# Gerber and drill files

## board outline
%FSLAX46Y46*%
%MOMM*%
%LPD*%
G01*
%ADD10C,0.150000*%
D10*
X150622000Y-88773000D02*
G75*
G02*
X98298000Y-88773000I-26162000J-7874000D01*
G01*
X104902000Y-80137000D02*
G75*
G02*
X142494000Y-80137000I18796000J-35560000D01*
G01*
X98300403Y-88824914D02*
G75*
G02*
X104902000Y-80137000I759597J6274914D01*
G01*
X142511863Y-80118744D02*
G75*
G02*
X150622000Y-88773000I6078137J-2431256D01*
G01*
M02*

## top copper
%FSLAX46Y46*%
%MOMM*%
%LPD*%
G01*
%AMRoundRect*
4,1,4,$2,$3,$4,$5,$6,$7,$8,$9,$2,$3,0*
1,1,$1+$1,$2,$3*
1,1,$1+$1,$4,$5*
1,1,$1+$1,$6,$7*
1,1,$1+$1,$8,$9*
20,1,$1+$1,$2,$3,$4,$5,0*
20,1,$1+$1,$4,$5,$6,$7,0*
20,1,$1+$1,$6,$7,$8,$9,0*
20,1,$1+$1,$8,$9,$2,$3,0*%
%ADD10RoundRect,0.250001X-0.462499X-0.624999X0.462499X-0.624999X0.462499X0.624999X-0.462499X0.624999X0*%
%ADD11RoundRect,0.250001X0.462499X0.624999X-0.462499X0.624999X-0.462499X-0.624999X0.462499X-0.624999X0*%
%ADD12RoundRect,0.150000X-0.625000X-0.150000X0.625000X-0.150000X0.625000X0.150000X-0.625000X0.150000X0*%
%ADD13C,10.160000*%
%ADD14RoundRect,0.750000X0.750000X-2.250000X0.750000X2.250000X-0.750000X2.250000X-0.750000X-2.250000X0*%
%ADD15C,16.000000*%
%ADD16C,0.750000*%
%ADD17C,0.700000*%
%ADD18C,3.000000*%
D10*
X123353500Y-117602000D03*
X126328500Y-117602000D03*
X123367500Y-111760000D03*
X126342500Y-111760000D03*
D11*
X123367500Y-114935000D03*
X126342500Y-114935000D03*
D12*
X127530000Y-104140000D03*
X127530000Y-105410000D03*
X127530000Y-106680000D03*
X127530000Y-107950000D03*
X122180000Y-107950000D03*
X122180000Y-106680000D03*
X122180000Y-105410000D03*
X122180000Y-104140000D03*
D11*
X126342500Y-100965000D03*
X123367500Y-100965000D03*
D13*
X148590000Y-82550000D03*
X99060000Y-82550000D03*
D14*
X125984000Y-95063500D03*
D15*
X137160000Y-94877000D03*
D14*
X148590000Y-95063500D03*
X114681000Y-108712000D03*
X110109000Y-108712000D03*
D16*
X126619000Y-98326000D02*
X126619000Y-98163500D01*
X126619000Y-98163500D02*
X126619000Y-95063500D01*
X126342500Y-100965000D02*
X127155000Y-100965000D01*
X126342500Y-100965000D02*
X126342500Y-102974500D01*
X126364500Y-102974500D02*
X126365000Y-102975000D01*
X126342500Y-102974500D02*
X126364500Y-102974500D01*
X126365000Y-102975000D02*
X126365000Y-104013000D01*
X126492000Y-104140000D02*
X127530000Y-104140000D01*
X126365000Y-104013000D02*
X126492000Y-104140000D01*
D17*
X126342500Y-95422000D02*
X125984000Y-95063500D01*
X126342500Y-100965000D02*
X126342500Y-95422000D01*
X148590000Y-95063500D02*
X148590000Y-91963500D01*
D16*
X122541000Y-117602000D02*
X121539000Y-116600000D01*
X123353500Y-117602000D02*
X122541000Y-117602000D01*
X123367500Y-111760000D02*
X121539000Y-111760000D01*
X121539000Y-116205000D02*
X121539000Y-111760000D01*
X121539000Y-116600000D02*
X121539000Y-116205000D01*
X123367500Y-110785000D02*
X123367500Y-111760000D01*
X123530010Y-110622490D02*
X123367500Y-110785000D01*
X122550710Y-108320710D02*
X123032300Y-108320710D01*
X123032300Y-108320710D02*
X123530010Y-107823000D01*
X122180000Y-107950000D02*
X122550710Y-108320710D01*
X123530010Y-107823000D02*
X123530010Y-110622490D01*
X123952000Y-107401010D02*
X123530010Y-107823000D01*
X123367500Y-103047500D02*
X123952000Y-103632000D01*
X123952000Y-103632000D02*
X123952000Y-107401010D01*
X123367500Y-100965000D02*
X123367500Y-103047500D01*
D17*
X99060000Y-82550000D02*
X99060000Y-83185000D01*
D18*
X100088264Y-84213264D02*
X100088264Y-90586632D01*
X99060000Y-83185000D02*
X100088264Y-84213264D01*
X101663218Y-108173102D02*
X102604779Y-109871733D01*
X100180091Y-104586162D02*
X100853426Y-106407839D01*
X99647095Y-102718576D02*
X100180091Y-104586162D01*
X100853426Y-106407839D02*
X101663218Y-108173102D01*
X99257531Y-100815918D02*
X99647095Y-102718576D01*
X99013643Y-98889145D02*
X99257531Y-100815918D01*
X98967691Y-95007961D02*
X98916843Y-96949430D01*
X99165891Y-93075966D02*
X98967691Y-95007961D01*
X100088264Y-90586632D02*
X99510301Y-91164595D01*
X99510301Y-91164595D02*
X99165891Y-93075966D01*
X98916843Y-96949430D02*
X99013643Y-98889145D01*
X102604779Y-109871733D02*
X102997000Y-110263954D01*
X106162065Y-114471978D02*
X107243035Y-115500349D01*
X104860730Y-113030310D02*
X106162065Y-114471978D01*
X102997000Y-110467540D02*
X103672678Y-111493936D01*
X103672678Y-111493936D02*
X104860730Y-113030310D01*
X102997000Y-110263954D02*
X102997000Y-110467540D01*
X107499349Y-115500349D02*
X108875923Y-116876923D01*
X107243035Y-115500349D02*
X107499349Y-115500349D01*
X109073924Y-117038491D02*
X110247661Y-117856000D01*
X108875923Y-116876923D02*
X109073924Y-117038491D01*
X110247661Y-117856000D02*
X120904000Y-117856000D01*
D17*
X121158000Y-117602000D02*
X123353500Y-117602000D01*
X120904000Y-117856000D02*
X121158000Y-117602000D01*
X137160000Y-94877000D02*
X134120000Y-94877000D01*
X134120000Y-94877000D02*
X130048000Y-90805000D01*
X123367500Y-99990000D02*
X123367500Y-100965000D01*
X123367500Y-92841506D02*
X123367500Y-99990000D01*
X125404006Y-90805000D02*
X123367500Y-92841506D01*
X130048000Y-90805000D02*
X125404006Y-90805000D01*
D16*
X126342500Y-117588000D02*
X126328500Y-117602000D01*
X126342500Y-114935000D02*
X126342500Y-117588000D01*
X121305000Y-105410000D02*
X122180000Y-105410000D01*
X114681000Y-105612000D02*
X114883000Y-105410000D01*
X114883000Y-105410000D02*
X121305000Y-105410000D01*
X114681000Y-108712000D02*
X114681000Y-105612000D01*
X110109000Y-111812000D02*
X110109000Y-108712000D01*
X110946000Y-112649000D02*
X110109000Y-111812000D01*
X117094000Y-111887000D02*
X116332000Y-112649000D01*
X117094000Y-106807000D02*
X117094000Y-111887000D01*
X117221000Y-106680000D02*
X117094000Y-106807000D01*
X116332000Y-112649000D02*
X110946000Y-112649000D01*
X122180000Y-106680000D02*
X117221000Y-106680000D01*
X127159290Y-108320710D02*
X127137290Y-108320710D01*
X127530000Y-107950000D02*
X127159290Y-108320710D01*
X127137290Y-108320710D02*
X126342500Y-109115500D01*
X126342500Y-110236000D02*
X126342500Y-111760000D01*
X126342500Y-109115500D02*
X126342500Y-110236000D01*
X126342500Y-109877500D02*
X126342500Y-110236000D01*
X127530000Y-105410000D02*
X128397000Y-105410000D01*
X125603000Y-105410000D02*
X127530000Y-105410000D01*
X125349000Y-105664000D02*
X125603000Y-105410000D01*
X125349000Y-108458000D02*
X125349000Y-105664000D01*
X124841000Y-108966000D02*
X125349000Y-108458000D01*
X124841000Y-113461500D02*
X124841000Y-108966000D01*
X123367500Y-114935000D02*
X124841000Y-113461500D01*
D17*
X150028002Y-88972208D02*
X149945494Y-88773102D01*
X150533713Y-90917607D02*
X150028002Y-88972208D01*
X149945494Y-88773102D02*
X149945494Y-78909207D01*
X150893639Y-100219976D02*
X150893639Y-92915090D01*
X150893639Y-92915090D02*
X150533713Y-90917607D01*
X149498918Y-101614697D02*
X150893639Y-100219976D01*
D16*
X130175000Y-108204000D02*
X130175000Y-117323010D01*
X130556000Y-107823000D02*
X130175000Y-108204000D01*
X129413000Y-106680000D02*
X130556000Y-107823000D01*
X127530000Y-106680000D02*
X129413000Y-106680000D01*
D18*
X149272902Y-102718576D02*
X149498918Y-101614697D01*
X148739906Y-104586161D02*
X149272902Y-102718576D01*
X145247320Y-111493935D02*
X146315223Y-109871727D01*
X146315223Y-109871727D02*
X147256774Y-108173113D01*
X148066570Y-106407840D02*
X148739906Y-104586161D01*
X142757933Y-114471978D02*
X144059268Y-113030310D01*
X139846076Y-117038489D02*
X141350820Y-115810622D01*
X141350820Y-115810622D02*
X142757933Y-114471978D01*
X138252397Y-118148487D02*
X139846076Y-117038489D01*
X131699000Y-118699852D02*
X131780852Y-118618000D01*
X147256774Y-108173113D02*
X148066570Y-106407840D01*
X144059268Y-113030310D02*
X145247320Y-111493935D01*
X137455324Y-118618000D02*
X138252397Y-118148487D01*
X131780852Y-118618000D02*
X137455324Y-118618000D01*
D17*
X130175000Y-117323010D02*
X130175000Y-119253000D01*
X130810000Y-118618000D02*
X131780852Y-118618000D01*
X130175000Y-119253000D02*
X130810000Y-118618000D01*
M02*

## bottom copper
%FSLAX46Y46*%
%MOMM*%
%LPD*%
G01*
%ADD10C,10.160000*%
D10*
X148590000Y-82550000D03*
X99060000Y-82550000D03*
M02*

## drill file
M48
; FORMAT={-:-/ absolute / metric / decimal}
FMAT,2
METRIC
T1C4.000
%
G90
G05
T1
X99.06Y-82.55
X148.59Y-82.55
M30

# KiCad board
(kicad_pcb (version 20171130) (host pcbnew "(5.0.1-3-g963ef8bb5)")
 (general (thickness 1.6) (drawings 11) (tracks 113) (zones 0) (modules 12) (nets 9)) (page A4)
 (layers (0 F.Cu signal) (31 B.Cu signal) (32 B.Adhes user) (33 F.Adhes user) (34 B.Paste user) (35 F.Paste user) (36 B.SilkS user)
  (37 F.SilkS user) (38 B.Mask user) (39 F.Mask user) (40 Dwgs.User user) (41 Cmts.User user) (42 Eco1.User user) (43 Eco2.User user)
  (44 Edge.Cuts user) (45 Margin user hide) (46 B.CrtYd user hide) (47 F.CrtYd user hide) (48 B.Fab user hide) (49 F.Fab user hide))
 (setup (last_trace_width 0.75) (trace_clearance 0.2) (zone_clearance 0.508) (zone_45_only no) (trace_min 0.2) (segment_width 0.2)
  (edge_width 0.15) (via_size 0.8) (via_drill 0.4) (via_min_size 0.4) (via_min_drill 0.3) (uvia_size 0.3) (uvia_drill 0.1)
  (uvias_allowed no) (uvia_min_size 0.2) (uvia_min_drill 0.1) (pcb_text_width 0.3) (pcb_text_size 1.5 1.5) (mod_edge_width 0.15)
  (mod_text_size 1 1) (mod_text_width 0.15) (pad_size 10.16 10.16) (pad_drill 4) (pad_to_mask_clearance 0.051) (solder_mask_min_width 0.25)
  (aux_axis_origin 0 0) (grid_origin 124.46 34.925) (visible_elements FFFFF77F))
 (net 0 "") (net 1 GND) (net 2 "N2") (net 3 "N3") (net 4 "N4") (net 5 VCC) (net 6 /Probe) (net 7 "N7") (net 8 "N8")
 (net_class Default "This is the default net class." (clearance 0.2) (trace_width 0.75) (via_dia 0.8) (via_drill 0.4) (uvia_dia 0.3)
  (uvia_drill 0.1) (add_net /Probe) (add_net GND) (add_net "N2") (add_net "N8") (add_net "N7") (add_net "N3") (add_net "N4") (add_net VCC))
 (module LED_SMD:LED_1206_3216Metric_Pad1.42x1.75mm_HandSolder (layer F.Cu) (at 124.841 117.602)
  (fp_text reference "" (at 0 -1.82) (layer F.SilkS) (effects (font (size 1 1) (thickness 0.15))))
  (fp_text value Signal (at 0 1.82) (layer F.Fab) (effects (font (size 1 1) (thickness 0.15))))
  (pad 1 smd roundrect (at -1.4875 0) (size 1.425 1.75) (layers F.Cu F.Paste F.Mask) (roundrect_rratio 0.175439) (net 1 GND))
  (pad 2 smd roundrect (at 1.4875 0) (size 1.425 1.75) (layers F.Cu F.Paste F.Mask) (roundrect_rratio 0.175439) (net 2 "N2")))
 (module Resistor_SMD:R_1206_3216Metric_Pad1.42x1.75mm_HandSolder (layer F.Cu) (at 124.855 111.76)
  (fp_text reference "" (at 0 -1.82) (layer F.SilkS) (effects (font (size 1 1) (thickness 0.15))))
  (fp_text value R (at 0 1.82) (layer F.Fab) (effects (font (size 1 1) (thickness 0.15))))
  (pad 1 smd roundrect (at -1.4875 0) (size 1.425 1.75) (layers F.Cu F.Paste F.Mask) (roundrect_rratio 0.175439) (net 1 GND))
  (pad 2 smd roundrect (at 1.4875 0) (size 1.425 1.75) (layers F.Cu F.Paste F.Mask) (roundrect_rratio 0.175439) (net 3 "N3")))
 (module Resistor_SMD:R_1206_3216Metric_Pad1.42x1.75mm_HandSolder (layer F.Cu) (at 124.855 114.935 180)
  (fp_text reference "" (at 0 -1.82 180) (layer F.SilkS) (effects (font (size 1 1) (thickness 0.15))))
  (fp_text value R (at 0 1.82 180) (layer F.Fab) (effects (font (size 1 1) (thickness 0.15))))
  (pad 2 smd roundrect (at 1.4875 0 180) (size 1.425 1.75) (layers F.Cu F.Paste F.Mask) (roundrect_rratio 0.175439) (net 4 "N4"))
  (pad 1 smd roundrect (at -1.4875 0 180) (size 1.425 1.75) (layers F.Cu F.Paste F.Mask) (roundrect_rratio 0.175439) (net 2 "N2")))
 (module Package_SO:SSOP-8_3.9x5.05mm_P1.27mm (layer F.Cu) (at 124.855 106.045)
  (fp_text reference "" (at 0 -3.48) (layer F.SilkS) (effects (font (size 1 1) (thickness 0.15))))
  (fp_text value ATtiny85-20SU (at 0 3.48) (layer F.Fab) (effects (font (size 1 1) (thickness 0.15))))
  (pad 8 smd roundrect (at 2.675 -1.905) (size 1.55 0.6) (layers F.Cu F.Paste F.Mask) (roundrect_rratio 0.25) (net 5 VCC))
  (pad 7 smd roundrect (at 2.675 -0.635) (size 1.55 0.6) (layers F.Cu F.Paste F.Mask) (roundrect_rratio 0.25) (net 4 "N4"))
  (pad 6 smd roundrect (at 2.675 0.635) (size 1.55 0.6) (layers F.Cu F.Paste F.Mask) (roundrect_rratio 0.25) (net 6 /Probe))
  (pad 5 smd roundrect (at 2.675 1.905) (size 1.55 0.6) (layers F.Cu F.Paste F.Mask) (roundrect_rratio 0.25) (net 3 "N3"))
  (pad 4 smd roundrect (at -2.675 1.905) (size 1.55 0.6) (layers F.Cu F.Paste F.Mask) (roundrect_rratio 0.25) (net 1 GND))
  (pad 3 smd roundrect (at -2.675 0.635) (size 1.55 0.6) (layers F.Cu F.Paste F.Mask) (roundrect_rratio 0.25) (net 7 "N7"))
  (pad 2 smd roundrect (at -2.675 -0.635) (size 1.55 0.6) (layers F.Cu F.Paste F.Mask) (roundrect_rratio 0.25) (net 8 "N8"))
  (pad 1 smd roundrect (at -2.675 -1.905) (size 1.55 0.6) (layers F.Cu F.Paste F.Mask) (roundrect_rratio 0.25)))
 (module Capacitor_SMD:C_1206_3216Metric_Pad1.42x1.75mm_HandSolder (layer F.Cu) (at 124.855 100.965 180)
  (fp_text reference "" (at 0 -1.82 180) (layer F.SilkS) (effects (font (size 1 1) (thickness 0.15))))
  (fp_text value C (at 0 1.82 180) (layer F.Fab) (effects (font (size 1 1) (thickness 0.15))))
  (pad 1 smd roundrect (at -1.4875 0 180) (size 1.425 1.75) (layers F.Cu F.Paste F.Mask) (roundrect_rratio 0.175439) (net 5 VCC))
  (pad 2 smd roundrect (at 1.4875 0 180) (size 1.425 1.75) (layers F.Cu F.Paste F.Mask) (roundrect_rratio 0.175439) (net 1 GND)))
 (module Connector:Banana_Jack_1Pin (layer F.Cu) (at 148.59 82.55)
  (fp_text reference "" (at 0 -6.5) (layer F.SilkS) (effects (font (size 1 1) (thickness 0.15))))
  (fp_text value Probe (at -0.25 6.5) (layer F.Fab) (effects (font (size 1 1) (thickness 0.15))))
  (pad 1 thru_hole circle (at 0 0) (size 10.16 10.16) (drill 4) (layers *.Cu *.Mask) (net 6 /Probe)))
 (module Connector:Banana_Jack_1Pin (layer F.Cu) (at 99.06 82.55)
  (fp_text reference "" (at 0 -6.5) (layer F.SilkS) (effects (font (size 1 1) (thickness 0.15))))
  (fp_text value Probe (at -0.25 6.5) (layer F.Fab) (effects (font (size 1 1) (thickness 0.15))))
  (pad 1 thru_hole circle (at 0 0) (size 10.16 10.16) (drill 4) (layers *.Cu *.Mask) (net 1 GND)))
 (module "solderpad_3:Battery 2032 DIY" (layer F.Cu) (at 137.16 95.0635)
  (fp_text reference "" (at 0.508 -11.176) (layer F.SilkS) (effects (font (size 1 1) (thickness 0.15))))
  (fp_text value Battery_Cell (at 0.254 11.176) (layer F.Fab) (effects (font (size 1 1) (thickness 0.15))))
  (pad 1 smd roundrect (at -11.176 0 90) (size 6 3) (layers F.Cu F.Paste F.Mask) (roundrect_rratio 0.25) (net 5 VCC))
  (pad 2 smd circle (at 0 -0.1865) (size 16 16) (layers F.Cu F.Paste F.Mask) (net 1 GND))
  (pad 1 smd roundrect (at 11.43 0 90) (size 6 3) (layers F.Cu F.Paste F.Mask) (roundrect_rratio 0.25) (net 5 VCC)))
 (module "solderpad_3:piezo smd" (layer F.Cu) (at 112.395 93.98 270)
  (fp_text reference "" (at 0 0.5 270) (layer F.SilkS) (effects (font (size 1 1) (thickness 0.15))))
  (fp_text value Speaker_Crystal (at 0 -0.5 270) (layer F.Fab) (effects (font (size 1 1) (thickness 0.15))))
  (pad 1 smd roundrect (at 14.732 -2.286 90) (size 6 3) (layers F.Cu F.Paste F.Mask) (roundrect_rratio 0.25) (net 8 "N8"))
  (pad 2 smd roundrect (at 14.732 2.286 90) (size 6 3) (layers F.Cu F.Paste F.Mask) (roundrect_rratio 0.25) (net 7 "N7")))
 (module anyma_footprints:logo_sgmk (layer F.Cu) (at 135.382 110.744)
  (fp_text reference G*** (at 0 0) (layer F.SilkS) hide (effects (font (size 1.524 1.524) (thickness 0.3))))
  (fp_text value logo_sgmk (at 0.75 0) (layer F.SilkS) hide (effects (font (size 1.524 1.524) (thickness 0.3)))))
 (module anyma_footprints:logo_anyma (layer B.Cu) (at 125.222 99.441 180)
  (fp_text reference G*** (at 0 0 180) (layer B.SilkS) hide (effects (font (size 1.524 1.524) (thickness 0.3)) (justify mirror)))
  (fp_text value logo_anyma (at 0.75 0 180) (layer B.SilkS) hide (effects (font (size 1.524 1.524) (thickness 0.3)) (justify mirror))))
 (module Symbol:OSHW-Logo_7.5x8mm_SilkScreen (layer B.Cu) (at 125.349 111.506 180)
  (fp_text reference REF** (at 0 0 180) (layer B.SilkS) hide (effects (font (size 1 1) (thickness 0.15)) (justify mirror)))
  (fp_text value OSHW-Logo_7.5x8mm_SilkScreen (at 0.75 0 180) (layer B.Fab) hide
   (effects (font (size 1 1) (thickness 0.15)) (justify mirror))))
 (gr_arc (start 124.46 96.647) (end 98.298 88.773) (angle -213.50053) (layer Edge.Cuts) (width 0.15))
 (gr_arc (start 123.698 115.697) (end 142.494 80.137) (angle -55.71930139) (layer Edge.Cuts) (width 0.15))
 (gr_arc (start 99.06 82.55) (end 104.902 80.137) (angle -240.6550052) (layer Edge.Cuts) (width 0.15))
 (gr_arc (start 148.59 82.55) (end 150.622 88.773) (angle -230.1151354) (layer Edge.Cuts) (width 0.15))
 (segment (start 126.619 98.326) (end 126.619 98.1635) (width 0.75) (layer F.Cu) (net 5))
 (segment (start 126.619 98.1635) (end 126.619 95.0635) (width 0.75) (layer F.Cu) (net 5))
 (segment (start 126.3425 100.965) (end 127.155 100.965) (width 0.75) (layer F.Cu) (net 5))
 (segment (start 126.3425 100.965) (end 126.3425 102.9745) (width 0.75) (layer F.Cu) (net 5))
 (segment (start 126.3645 102.9745) (end 126.365 102.975) (width 0.75) (layer F.Cu) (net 5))
 (segment (start 126.3425 102.9745) (end 126.3645 102.9745) (width 0.75) (layer F.Cu) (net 5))
 (segment (start 126.365 102.975) (end 126.365 104.013) (width 0.75) (layer F.Cu) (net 5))
 (segment (start 126.492 104.14) (end 127.53 104.14) (width 0.75) (layer F.Cu) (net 5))
 (segment (start 126.365 104.013) (end 126.492 104.14) (width 0.75) (layer F.Cu) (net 5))
 (segment (start 126.3425 95.422) (end 125.984 95.0635) (width 0.7) (layer F.Cu) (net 5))
 (segment (start 126.3425 100.965) (end 126.3425 95.422) (width 0.7) (layer F.Cu) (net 5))
 (segment (start 148.59 95.0635) (end 148.59 91.9635) (width 0.7) (layer F.Cu) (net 5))
 (segment (start 122.541 117.602) (end 121.539 116.6) (width 0.75) (layer F.Cu) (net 1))
 (segment (start 123.3535 117.602) (end 122.541 117.602) (width 0.75) (layer F.Cu) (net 1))
 (segment (start 123.3675 111.76) (end 121.539 111.76) (width 0.75) (layer F.Cu) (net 1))
 (segment (start 121.539 116.205) (end 121.539 111.76) (width 0.75) (layer F.Cu) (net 1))
 (segment (start 121.539 116.6) (end 121.539 116.205) (width 0.75) (layer F.Cu) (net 1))
 (segment (start 123.3675 110.785) (end 123.3675 111.76) (width 0.75) (layer F.Cu) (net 1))
 (segment (start 123.53001 110.62249) (end 123.3675 110.785) (width 0.75) (layer F.Cu) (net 1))
 (segment (start 122.55071 108.32071) (end 123.0323 108.32071) (width 0.75) (layer F.Cu) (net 1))
 (segment (start 123.0323 108.32071) (end 123.53001 107.823) (width 0.75) (layer F.Cu) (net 1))
 (segment (start 122.18 107.95) (end 122.55071 108.32071) (width 0.75) (layer F.Cu) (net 1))
 (segment (start 123.53001 107.823) (end 123.53001 110.62249) (width 0.75) (layer F.Cu) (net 1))
 (segment (start 123.952 107.40101) (end 123.53001 107.823) (width 0.75) (layer F.Cu) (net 1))
 (segment (start 123.3675 103.0475) (end 123.952 103.632) (width 0.75) (layer F.Cu) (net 1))
 (segment (start 123.952 103.632) (end 123.952 107.40101) (width 0.75) (layer F.Cu) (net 1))
 (segment (start 123.3675 100.965) (end 123.3675 103.0475) (width 0.75) (layer F.Cu) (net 1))
 (segment (start 99.06 82.55) (end 99.06 83.185) (width 0.7) (layer F.Cu) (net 1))
 (segment (start 100.088264 84.213264) (end 100.088264 90.586632) (width 3) (layer F.Cu) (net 1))
 (segment (start 99.06 83.185) (end 100.088264 84.213264) (width 3) (layer F.Cu) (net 1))
 (segment (start 101.663218 108.173102) (end 102.604779 109.871733) (width 3) (layer F.Cu) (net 1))
 (segment (start 100.180091 104.586162) (end 100.853426 106.407839) (width 3) (layer F.Cu) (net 1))
 (segment (start 99.647095 102.718576) (end 100.180091 104.586162) (width 3) (layer F.Cu) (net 1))
 (segment (start 100.853426 106.407839) (end 101.663218 108.173102) (width 3) (layer F.Cu) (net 1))
 (segment (start 99.257531 100.815918) (end 99.647095 102.718576) (width 3) (layer F.Cu) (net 1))
 (segment (start 99.013643 98.889145) (end 99.257531 100.815918) (width 3) (layer F.Cu) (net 1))
 (segment (start 98.967691 95.007961) (end 98.916843 96.94943) (width 3) (layer F.Cu) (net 1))
 (segment (start 99.165891 93.075966) (end 98.967691 95.007961) (width 3) (layer F.Cu) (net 1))
 (segment (start 100.088264 90.586632) (end 99.510301 91.164595) (width 3) (layer F.Cu) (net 1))
 (segment (start 99.510301 91.164595) (end 99.165891 93.075966) (width 3) (layer F.Cu) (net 1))
 (segment (start 98.916843 96.94943) (end 99.013643 98.889145) (width 3) (layer F.Cu) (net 1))
 (segment (start 102.604779 109.871733) (end 102.997 110.263954) (width 3) (layer F.Cu) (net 1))
 (segment (start 106.162065 114.471978) (end 107.243035 115.500349) (width 3) (layer F.Cu) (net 1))
 (segment (start 104.86073 113.03031) (end 106.162065 114.471978) (width 3) (layer F.Cu) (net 1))
 (segment (start 102.997 110.46754) (end 103.672678 111.493936) (width 3) (layer F.Cu) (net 1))
 (segment (start 103.672678 111.493936) (end 104.86073 113.03031) (width 3) (layer F.Cu) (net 1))
 (segment (start 102.997 110.263954) (end 102.997 110.46754) (width 3) (layer F.Cu) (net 1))
 (segment (start 107.499349 115.500349) (end 108.875923 116.876923) (width 3) (layer F.Cu) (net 1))
 (segment (start 107.243035 115.500349) (end 107.499349 115.500349) (width 3) (layer F.Cu) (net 1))
 (segment (start 109.073924 117.038491) (end 110.247661 117.856) (width 3) (layer F.Cu) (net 1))
 (segment (start 108.875923 116.876923) (end 109.073924 117.038491) (width 3) (layer F.Cu) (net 1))
 (segment (start 110.247661 117.856) (end 120.904 117.856) (width 3) (layer F.Cu) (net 1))
 (segment (start 121.158 117.602) (end 123.3535 117.602) (width 0.7) (layer F.Cu) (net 1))
 (segment (start 120.904 117.856) (end 121.158 117.602) (width 0.7) (layer F.Cu) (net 1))
 (segment (start 137.16 94.877) (end 134.12 94.877) (width 0.7) (layer F.Cu) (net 1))
 (segment (start 134.12 94.877) (end 130.048 90.805) (width 0.7) (layer F.Cu) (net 1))
 (segment (start 123.3675 99.99) (end 123.3675 100.965) (width 0.7) (layer F.Cu) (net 1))
 (segment (start 123.3675 92.841506) (end 123.3675 99.99) (width 0.7) (layer F.Cu) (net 1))
 (segment (start 125.404006 90.805) (end 123.3675 92.841506) (width 0.7) (layer F.Cu) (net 1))
 (segment (start 130.048 90.805) (end 125.404006 90.805) (width 0.7) (layer F.Cu) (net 1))
 (segment (start 126.3425 117.588) (end 126.3285 117.602) (width 0.75) (layer F.Cu) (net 2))
 (segment (start 126.3425 114.935) (end 126.3425 117.588) (width 0.75) (layer F.Cu) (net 2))
 (segment (start 121.305 105.41) (end 122.18 105.41) (width 0.75) (layer F.Cu) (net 8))
 (segment (start 114.681 105.612) (end 114.883 105.41) (width 0.75) (layer F.Cu) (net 8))
 (segment (start 114.883 105.41) (end 121.305 105.41) (width 0.75) (layer F.Cu) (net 8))
 (segment (start 114.681 108.712) (end 114.681 105.612) (width 0.75) (layer F.Cu) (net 8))
 (segment (start 110.109 111.812) (end 110.109 108.712) (width 0.75) (layer F.Cu) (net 7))
 (segment (start 110.946 112.649) (end 110.109 111.812) (width 0.75) (layer F.Cu) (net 7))
 (segment (start 117.094 111.887) (end 116.332 112.649) (width 0.75) (layer F.Cu) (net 7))
 (segment (start 117.094 106.807) (end 117.094 111.887) (width 0.75) (layer F.Cu) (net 7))
 (segment (start 117.221 106.68) (end 117.094 106.807) (width 0.75) (layer F.Cu) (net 7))
 (segment (start 116.332 112.649) (end 110.946 112.649) (width 0.75) (layer F.Cu) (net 7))
 (segment (start 122.18 106.68) (end 117.221 106.68) (width 0.75) (layer F.Cu) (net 7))
 (segment (start 127.15929 108.32071) (end 127.13729 108.32071) (width 0.75) (layer F.Cu) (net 3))
 (segment (start 127.53 107.95) (end 127.15929 108.32071) (width 0.75) (layer F.Cu) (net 3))
 (segment (start 127.13729 108.32071) (end 126.3425 109.1155) (width 0.75) (layer F.Cu) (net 3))
 (segment (start 126.3425 110.236) (end 126.3425 111.76) (width 0.75) (layer F.Cu) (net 3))
 (segment (start 126.3425 109.1155) (end 126.3425 110.236) (width 0.75) (layer F.Cu) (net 3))
 (segment (start 126.3425 109.8775) (end 126.3425 110.236) (width 0.75) (layer F.Cu) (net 3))
 (segment (start 127.53 105.41) (end 128.397 105.41) (width 0.75) (layer F.Cu) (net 4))
 (segment (start 125.603 105.41) (end 127.53 105.41) (width 0.75) (layer F.Cu) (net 4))
 (segment (start 125.349 105.664) (end 125.603 105.41) (width 0.75) (layer F.Cu) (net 4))
 (segment (start 125.349 108.458) (end 125.349 105.664) (width 0.75) (layer F.Cu) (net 4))
 (segment (start 124.841 108.966) (end 125.349 108.458) (width 0.75) (layer F.Cu) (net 4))
 (segment (start 124.841 113.4615) (end 124.841 108.966) (width 0.75) (layer F.Cu) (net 4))
 (segment (start 123.3675 114.935) (end 124.841 113.4615) (width 0.75) (layer F.Cu) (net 4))
 (segment (start 150.028002 88.972208) (end 149.945494 88.773102) (width 0.7) (layer F.Cu) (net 6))
 (segment (start 150.533713 90.917607) (end 150.028002 88.972208) (width 0.7) (layer F.Cu) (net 6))
 (segment (start 149.945494 88.773102) (end 149.945494 78.909207) (width 0.7) (layer F.Cu) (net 6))
 (segment (start 150.893639 100.219976) (end 150.893639 92.91509) (width 0.7) (layer F.Cu) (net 6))
 (segment (start 150.893639 92.91509) (end 150.533713 90.917607) (width 0.7) (layer F.Cu) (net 6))
 (segment (start 149.498918 101.614697) (end 150.893639 100.219976) (width 0.7) (layer F.Cu) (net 6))
 (segment (start 130.175 108.204) (end 130.175 117.32301) (width 0.75) (layer F.Cu) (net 6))
 (segment (start 130.556 107.823) (end 130.175 108.204) (width 0.75) (layer F.Cu) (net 6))
 (segment (start 129.413 106.68) (end 130.556 107.823) (width 0.75) (layer F.Cu) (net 6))
 (segment (start 127.53 106.68) (end 129.413 106.68) (width 0.75) (layer F.Cu) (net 6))
 (segment (start 149.272902 102.718576) (end 149.498918 101.614697) (width 3) (layer F.Cu) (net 6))
 (segment (start 148.739906 104.586161) (end 149.272902 102.718576) (width 3) (layer F.Cu) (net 6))
 (segment (start 145.24732 111.493935) (end 146.315223 109.871727) (width 3) (layer F.Cu) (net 6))
 (segment (start 146.315223 109.871727) (end 147.256774 108.173113) (width 3) (layer F.Cu) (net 6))
 (segment (start 148.06657 106.40784) (end 148.739906 104.586161) (width 3) (layer F.Cu) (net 6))
 (segment (start 142.757933 114.471978) (end 144.059268 113.03031) (width 3) (layer F.Cu) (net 6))
 (segment (start 139.846076 117.038489) (end 141.35082 115.810622) (width 3) (layer F.Cu) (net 6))
 (segment (start 141.35082 115.810622) (end 142.757933 114.471978) (width 3) (layer F.Cu) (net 6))
 (segment (start 138.252397 118.148487) (end 139.846076 117.038489) (width 3) (layer F.Cu) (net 6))
 (segment (start 131.699 118.699852) (end 131.780852 118.618) (width 3) (layer F.Cu) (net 6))
 (segment (start 147.256774 108.173113) (end 148.06657 106.40784) (width 3) (layer F.Cu) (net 6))
 (segment (start 144.059268 113.03031) (end 145.24732 111.493935) (width 3) (layer F.Cu) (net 6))
 (segment (start 137.455324 118.618) (end 138.252397 118.148487) (width 3) (layer F.Cu) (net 6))
 (segment (start 131.780852 118.618) (end 137.455324 118.618) (width 3) (layer F.Cu) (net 6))
 (segment (start 130.175 117.32301) (end 130.175 119.253) (width 0.7) (layer F.Cu) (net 6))
 (segment (start 130.81 118.618) (end 131.780852 118.618) (width 0.7) (layer F.Cu) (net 6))
 (segment (start 130.175 119.253) (end 130.81 118.618) (width 0.7) (layer F.Cu) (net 6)))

